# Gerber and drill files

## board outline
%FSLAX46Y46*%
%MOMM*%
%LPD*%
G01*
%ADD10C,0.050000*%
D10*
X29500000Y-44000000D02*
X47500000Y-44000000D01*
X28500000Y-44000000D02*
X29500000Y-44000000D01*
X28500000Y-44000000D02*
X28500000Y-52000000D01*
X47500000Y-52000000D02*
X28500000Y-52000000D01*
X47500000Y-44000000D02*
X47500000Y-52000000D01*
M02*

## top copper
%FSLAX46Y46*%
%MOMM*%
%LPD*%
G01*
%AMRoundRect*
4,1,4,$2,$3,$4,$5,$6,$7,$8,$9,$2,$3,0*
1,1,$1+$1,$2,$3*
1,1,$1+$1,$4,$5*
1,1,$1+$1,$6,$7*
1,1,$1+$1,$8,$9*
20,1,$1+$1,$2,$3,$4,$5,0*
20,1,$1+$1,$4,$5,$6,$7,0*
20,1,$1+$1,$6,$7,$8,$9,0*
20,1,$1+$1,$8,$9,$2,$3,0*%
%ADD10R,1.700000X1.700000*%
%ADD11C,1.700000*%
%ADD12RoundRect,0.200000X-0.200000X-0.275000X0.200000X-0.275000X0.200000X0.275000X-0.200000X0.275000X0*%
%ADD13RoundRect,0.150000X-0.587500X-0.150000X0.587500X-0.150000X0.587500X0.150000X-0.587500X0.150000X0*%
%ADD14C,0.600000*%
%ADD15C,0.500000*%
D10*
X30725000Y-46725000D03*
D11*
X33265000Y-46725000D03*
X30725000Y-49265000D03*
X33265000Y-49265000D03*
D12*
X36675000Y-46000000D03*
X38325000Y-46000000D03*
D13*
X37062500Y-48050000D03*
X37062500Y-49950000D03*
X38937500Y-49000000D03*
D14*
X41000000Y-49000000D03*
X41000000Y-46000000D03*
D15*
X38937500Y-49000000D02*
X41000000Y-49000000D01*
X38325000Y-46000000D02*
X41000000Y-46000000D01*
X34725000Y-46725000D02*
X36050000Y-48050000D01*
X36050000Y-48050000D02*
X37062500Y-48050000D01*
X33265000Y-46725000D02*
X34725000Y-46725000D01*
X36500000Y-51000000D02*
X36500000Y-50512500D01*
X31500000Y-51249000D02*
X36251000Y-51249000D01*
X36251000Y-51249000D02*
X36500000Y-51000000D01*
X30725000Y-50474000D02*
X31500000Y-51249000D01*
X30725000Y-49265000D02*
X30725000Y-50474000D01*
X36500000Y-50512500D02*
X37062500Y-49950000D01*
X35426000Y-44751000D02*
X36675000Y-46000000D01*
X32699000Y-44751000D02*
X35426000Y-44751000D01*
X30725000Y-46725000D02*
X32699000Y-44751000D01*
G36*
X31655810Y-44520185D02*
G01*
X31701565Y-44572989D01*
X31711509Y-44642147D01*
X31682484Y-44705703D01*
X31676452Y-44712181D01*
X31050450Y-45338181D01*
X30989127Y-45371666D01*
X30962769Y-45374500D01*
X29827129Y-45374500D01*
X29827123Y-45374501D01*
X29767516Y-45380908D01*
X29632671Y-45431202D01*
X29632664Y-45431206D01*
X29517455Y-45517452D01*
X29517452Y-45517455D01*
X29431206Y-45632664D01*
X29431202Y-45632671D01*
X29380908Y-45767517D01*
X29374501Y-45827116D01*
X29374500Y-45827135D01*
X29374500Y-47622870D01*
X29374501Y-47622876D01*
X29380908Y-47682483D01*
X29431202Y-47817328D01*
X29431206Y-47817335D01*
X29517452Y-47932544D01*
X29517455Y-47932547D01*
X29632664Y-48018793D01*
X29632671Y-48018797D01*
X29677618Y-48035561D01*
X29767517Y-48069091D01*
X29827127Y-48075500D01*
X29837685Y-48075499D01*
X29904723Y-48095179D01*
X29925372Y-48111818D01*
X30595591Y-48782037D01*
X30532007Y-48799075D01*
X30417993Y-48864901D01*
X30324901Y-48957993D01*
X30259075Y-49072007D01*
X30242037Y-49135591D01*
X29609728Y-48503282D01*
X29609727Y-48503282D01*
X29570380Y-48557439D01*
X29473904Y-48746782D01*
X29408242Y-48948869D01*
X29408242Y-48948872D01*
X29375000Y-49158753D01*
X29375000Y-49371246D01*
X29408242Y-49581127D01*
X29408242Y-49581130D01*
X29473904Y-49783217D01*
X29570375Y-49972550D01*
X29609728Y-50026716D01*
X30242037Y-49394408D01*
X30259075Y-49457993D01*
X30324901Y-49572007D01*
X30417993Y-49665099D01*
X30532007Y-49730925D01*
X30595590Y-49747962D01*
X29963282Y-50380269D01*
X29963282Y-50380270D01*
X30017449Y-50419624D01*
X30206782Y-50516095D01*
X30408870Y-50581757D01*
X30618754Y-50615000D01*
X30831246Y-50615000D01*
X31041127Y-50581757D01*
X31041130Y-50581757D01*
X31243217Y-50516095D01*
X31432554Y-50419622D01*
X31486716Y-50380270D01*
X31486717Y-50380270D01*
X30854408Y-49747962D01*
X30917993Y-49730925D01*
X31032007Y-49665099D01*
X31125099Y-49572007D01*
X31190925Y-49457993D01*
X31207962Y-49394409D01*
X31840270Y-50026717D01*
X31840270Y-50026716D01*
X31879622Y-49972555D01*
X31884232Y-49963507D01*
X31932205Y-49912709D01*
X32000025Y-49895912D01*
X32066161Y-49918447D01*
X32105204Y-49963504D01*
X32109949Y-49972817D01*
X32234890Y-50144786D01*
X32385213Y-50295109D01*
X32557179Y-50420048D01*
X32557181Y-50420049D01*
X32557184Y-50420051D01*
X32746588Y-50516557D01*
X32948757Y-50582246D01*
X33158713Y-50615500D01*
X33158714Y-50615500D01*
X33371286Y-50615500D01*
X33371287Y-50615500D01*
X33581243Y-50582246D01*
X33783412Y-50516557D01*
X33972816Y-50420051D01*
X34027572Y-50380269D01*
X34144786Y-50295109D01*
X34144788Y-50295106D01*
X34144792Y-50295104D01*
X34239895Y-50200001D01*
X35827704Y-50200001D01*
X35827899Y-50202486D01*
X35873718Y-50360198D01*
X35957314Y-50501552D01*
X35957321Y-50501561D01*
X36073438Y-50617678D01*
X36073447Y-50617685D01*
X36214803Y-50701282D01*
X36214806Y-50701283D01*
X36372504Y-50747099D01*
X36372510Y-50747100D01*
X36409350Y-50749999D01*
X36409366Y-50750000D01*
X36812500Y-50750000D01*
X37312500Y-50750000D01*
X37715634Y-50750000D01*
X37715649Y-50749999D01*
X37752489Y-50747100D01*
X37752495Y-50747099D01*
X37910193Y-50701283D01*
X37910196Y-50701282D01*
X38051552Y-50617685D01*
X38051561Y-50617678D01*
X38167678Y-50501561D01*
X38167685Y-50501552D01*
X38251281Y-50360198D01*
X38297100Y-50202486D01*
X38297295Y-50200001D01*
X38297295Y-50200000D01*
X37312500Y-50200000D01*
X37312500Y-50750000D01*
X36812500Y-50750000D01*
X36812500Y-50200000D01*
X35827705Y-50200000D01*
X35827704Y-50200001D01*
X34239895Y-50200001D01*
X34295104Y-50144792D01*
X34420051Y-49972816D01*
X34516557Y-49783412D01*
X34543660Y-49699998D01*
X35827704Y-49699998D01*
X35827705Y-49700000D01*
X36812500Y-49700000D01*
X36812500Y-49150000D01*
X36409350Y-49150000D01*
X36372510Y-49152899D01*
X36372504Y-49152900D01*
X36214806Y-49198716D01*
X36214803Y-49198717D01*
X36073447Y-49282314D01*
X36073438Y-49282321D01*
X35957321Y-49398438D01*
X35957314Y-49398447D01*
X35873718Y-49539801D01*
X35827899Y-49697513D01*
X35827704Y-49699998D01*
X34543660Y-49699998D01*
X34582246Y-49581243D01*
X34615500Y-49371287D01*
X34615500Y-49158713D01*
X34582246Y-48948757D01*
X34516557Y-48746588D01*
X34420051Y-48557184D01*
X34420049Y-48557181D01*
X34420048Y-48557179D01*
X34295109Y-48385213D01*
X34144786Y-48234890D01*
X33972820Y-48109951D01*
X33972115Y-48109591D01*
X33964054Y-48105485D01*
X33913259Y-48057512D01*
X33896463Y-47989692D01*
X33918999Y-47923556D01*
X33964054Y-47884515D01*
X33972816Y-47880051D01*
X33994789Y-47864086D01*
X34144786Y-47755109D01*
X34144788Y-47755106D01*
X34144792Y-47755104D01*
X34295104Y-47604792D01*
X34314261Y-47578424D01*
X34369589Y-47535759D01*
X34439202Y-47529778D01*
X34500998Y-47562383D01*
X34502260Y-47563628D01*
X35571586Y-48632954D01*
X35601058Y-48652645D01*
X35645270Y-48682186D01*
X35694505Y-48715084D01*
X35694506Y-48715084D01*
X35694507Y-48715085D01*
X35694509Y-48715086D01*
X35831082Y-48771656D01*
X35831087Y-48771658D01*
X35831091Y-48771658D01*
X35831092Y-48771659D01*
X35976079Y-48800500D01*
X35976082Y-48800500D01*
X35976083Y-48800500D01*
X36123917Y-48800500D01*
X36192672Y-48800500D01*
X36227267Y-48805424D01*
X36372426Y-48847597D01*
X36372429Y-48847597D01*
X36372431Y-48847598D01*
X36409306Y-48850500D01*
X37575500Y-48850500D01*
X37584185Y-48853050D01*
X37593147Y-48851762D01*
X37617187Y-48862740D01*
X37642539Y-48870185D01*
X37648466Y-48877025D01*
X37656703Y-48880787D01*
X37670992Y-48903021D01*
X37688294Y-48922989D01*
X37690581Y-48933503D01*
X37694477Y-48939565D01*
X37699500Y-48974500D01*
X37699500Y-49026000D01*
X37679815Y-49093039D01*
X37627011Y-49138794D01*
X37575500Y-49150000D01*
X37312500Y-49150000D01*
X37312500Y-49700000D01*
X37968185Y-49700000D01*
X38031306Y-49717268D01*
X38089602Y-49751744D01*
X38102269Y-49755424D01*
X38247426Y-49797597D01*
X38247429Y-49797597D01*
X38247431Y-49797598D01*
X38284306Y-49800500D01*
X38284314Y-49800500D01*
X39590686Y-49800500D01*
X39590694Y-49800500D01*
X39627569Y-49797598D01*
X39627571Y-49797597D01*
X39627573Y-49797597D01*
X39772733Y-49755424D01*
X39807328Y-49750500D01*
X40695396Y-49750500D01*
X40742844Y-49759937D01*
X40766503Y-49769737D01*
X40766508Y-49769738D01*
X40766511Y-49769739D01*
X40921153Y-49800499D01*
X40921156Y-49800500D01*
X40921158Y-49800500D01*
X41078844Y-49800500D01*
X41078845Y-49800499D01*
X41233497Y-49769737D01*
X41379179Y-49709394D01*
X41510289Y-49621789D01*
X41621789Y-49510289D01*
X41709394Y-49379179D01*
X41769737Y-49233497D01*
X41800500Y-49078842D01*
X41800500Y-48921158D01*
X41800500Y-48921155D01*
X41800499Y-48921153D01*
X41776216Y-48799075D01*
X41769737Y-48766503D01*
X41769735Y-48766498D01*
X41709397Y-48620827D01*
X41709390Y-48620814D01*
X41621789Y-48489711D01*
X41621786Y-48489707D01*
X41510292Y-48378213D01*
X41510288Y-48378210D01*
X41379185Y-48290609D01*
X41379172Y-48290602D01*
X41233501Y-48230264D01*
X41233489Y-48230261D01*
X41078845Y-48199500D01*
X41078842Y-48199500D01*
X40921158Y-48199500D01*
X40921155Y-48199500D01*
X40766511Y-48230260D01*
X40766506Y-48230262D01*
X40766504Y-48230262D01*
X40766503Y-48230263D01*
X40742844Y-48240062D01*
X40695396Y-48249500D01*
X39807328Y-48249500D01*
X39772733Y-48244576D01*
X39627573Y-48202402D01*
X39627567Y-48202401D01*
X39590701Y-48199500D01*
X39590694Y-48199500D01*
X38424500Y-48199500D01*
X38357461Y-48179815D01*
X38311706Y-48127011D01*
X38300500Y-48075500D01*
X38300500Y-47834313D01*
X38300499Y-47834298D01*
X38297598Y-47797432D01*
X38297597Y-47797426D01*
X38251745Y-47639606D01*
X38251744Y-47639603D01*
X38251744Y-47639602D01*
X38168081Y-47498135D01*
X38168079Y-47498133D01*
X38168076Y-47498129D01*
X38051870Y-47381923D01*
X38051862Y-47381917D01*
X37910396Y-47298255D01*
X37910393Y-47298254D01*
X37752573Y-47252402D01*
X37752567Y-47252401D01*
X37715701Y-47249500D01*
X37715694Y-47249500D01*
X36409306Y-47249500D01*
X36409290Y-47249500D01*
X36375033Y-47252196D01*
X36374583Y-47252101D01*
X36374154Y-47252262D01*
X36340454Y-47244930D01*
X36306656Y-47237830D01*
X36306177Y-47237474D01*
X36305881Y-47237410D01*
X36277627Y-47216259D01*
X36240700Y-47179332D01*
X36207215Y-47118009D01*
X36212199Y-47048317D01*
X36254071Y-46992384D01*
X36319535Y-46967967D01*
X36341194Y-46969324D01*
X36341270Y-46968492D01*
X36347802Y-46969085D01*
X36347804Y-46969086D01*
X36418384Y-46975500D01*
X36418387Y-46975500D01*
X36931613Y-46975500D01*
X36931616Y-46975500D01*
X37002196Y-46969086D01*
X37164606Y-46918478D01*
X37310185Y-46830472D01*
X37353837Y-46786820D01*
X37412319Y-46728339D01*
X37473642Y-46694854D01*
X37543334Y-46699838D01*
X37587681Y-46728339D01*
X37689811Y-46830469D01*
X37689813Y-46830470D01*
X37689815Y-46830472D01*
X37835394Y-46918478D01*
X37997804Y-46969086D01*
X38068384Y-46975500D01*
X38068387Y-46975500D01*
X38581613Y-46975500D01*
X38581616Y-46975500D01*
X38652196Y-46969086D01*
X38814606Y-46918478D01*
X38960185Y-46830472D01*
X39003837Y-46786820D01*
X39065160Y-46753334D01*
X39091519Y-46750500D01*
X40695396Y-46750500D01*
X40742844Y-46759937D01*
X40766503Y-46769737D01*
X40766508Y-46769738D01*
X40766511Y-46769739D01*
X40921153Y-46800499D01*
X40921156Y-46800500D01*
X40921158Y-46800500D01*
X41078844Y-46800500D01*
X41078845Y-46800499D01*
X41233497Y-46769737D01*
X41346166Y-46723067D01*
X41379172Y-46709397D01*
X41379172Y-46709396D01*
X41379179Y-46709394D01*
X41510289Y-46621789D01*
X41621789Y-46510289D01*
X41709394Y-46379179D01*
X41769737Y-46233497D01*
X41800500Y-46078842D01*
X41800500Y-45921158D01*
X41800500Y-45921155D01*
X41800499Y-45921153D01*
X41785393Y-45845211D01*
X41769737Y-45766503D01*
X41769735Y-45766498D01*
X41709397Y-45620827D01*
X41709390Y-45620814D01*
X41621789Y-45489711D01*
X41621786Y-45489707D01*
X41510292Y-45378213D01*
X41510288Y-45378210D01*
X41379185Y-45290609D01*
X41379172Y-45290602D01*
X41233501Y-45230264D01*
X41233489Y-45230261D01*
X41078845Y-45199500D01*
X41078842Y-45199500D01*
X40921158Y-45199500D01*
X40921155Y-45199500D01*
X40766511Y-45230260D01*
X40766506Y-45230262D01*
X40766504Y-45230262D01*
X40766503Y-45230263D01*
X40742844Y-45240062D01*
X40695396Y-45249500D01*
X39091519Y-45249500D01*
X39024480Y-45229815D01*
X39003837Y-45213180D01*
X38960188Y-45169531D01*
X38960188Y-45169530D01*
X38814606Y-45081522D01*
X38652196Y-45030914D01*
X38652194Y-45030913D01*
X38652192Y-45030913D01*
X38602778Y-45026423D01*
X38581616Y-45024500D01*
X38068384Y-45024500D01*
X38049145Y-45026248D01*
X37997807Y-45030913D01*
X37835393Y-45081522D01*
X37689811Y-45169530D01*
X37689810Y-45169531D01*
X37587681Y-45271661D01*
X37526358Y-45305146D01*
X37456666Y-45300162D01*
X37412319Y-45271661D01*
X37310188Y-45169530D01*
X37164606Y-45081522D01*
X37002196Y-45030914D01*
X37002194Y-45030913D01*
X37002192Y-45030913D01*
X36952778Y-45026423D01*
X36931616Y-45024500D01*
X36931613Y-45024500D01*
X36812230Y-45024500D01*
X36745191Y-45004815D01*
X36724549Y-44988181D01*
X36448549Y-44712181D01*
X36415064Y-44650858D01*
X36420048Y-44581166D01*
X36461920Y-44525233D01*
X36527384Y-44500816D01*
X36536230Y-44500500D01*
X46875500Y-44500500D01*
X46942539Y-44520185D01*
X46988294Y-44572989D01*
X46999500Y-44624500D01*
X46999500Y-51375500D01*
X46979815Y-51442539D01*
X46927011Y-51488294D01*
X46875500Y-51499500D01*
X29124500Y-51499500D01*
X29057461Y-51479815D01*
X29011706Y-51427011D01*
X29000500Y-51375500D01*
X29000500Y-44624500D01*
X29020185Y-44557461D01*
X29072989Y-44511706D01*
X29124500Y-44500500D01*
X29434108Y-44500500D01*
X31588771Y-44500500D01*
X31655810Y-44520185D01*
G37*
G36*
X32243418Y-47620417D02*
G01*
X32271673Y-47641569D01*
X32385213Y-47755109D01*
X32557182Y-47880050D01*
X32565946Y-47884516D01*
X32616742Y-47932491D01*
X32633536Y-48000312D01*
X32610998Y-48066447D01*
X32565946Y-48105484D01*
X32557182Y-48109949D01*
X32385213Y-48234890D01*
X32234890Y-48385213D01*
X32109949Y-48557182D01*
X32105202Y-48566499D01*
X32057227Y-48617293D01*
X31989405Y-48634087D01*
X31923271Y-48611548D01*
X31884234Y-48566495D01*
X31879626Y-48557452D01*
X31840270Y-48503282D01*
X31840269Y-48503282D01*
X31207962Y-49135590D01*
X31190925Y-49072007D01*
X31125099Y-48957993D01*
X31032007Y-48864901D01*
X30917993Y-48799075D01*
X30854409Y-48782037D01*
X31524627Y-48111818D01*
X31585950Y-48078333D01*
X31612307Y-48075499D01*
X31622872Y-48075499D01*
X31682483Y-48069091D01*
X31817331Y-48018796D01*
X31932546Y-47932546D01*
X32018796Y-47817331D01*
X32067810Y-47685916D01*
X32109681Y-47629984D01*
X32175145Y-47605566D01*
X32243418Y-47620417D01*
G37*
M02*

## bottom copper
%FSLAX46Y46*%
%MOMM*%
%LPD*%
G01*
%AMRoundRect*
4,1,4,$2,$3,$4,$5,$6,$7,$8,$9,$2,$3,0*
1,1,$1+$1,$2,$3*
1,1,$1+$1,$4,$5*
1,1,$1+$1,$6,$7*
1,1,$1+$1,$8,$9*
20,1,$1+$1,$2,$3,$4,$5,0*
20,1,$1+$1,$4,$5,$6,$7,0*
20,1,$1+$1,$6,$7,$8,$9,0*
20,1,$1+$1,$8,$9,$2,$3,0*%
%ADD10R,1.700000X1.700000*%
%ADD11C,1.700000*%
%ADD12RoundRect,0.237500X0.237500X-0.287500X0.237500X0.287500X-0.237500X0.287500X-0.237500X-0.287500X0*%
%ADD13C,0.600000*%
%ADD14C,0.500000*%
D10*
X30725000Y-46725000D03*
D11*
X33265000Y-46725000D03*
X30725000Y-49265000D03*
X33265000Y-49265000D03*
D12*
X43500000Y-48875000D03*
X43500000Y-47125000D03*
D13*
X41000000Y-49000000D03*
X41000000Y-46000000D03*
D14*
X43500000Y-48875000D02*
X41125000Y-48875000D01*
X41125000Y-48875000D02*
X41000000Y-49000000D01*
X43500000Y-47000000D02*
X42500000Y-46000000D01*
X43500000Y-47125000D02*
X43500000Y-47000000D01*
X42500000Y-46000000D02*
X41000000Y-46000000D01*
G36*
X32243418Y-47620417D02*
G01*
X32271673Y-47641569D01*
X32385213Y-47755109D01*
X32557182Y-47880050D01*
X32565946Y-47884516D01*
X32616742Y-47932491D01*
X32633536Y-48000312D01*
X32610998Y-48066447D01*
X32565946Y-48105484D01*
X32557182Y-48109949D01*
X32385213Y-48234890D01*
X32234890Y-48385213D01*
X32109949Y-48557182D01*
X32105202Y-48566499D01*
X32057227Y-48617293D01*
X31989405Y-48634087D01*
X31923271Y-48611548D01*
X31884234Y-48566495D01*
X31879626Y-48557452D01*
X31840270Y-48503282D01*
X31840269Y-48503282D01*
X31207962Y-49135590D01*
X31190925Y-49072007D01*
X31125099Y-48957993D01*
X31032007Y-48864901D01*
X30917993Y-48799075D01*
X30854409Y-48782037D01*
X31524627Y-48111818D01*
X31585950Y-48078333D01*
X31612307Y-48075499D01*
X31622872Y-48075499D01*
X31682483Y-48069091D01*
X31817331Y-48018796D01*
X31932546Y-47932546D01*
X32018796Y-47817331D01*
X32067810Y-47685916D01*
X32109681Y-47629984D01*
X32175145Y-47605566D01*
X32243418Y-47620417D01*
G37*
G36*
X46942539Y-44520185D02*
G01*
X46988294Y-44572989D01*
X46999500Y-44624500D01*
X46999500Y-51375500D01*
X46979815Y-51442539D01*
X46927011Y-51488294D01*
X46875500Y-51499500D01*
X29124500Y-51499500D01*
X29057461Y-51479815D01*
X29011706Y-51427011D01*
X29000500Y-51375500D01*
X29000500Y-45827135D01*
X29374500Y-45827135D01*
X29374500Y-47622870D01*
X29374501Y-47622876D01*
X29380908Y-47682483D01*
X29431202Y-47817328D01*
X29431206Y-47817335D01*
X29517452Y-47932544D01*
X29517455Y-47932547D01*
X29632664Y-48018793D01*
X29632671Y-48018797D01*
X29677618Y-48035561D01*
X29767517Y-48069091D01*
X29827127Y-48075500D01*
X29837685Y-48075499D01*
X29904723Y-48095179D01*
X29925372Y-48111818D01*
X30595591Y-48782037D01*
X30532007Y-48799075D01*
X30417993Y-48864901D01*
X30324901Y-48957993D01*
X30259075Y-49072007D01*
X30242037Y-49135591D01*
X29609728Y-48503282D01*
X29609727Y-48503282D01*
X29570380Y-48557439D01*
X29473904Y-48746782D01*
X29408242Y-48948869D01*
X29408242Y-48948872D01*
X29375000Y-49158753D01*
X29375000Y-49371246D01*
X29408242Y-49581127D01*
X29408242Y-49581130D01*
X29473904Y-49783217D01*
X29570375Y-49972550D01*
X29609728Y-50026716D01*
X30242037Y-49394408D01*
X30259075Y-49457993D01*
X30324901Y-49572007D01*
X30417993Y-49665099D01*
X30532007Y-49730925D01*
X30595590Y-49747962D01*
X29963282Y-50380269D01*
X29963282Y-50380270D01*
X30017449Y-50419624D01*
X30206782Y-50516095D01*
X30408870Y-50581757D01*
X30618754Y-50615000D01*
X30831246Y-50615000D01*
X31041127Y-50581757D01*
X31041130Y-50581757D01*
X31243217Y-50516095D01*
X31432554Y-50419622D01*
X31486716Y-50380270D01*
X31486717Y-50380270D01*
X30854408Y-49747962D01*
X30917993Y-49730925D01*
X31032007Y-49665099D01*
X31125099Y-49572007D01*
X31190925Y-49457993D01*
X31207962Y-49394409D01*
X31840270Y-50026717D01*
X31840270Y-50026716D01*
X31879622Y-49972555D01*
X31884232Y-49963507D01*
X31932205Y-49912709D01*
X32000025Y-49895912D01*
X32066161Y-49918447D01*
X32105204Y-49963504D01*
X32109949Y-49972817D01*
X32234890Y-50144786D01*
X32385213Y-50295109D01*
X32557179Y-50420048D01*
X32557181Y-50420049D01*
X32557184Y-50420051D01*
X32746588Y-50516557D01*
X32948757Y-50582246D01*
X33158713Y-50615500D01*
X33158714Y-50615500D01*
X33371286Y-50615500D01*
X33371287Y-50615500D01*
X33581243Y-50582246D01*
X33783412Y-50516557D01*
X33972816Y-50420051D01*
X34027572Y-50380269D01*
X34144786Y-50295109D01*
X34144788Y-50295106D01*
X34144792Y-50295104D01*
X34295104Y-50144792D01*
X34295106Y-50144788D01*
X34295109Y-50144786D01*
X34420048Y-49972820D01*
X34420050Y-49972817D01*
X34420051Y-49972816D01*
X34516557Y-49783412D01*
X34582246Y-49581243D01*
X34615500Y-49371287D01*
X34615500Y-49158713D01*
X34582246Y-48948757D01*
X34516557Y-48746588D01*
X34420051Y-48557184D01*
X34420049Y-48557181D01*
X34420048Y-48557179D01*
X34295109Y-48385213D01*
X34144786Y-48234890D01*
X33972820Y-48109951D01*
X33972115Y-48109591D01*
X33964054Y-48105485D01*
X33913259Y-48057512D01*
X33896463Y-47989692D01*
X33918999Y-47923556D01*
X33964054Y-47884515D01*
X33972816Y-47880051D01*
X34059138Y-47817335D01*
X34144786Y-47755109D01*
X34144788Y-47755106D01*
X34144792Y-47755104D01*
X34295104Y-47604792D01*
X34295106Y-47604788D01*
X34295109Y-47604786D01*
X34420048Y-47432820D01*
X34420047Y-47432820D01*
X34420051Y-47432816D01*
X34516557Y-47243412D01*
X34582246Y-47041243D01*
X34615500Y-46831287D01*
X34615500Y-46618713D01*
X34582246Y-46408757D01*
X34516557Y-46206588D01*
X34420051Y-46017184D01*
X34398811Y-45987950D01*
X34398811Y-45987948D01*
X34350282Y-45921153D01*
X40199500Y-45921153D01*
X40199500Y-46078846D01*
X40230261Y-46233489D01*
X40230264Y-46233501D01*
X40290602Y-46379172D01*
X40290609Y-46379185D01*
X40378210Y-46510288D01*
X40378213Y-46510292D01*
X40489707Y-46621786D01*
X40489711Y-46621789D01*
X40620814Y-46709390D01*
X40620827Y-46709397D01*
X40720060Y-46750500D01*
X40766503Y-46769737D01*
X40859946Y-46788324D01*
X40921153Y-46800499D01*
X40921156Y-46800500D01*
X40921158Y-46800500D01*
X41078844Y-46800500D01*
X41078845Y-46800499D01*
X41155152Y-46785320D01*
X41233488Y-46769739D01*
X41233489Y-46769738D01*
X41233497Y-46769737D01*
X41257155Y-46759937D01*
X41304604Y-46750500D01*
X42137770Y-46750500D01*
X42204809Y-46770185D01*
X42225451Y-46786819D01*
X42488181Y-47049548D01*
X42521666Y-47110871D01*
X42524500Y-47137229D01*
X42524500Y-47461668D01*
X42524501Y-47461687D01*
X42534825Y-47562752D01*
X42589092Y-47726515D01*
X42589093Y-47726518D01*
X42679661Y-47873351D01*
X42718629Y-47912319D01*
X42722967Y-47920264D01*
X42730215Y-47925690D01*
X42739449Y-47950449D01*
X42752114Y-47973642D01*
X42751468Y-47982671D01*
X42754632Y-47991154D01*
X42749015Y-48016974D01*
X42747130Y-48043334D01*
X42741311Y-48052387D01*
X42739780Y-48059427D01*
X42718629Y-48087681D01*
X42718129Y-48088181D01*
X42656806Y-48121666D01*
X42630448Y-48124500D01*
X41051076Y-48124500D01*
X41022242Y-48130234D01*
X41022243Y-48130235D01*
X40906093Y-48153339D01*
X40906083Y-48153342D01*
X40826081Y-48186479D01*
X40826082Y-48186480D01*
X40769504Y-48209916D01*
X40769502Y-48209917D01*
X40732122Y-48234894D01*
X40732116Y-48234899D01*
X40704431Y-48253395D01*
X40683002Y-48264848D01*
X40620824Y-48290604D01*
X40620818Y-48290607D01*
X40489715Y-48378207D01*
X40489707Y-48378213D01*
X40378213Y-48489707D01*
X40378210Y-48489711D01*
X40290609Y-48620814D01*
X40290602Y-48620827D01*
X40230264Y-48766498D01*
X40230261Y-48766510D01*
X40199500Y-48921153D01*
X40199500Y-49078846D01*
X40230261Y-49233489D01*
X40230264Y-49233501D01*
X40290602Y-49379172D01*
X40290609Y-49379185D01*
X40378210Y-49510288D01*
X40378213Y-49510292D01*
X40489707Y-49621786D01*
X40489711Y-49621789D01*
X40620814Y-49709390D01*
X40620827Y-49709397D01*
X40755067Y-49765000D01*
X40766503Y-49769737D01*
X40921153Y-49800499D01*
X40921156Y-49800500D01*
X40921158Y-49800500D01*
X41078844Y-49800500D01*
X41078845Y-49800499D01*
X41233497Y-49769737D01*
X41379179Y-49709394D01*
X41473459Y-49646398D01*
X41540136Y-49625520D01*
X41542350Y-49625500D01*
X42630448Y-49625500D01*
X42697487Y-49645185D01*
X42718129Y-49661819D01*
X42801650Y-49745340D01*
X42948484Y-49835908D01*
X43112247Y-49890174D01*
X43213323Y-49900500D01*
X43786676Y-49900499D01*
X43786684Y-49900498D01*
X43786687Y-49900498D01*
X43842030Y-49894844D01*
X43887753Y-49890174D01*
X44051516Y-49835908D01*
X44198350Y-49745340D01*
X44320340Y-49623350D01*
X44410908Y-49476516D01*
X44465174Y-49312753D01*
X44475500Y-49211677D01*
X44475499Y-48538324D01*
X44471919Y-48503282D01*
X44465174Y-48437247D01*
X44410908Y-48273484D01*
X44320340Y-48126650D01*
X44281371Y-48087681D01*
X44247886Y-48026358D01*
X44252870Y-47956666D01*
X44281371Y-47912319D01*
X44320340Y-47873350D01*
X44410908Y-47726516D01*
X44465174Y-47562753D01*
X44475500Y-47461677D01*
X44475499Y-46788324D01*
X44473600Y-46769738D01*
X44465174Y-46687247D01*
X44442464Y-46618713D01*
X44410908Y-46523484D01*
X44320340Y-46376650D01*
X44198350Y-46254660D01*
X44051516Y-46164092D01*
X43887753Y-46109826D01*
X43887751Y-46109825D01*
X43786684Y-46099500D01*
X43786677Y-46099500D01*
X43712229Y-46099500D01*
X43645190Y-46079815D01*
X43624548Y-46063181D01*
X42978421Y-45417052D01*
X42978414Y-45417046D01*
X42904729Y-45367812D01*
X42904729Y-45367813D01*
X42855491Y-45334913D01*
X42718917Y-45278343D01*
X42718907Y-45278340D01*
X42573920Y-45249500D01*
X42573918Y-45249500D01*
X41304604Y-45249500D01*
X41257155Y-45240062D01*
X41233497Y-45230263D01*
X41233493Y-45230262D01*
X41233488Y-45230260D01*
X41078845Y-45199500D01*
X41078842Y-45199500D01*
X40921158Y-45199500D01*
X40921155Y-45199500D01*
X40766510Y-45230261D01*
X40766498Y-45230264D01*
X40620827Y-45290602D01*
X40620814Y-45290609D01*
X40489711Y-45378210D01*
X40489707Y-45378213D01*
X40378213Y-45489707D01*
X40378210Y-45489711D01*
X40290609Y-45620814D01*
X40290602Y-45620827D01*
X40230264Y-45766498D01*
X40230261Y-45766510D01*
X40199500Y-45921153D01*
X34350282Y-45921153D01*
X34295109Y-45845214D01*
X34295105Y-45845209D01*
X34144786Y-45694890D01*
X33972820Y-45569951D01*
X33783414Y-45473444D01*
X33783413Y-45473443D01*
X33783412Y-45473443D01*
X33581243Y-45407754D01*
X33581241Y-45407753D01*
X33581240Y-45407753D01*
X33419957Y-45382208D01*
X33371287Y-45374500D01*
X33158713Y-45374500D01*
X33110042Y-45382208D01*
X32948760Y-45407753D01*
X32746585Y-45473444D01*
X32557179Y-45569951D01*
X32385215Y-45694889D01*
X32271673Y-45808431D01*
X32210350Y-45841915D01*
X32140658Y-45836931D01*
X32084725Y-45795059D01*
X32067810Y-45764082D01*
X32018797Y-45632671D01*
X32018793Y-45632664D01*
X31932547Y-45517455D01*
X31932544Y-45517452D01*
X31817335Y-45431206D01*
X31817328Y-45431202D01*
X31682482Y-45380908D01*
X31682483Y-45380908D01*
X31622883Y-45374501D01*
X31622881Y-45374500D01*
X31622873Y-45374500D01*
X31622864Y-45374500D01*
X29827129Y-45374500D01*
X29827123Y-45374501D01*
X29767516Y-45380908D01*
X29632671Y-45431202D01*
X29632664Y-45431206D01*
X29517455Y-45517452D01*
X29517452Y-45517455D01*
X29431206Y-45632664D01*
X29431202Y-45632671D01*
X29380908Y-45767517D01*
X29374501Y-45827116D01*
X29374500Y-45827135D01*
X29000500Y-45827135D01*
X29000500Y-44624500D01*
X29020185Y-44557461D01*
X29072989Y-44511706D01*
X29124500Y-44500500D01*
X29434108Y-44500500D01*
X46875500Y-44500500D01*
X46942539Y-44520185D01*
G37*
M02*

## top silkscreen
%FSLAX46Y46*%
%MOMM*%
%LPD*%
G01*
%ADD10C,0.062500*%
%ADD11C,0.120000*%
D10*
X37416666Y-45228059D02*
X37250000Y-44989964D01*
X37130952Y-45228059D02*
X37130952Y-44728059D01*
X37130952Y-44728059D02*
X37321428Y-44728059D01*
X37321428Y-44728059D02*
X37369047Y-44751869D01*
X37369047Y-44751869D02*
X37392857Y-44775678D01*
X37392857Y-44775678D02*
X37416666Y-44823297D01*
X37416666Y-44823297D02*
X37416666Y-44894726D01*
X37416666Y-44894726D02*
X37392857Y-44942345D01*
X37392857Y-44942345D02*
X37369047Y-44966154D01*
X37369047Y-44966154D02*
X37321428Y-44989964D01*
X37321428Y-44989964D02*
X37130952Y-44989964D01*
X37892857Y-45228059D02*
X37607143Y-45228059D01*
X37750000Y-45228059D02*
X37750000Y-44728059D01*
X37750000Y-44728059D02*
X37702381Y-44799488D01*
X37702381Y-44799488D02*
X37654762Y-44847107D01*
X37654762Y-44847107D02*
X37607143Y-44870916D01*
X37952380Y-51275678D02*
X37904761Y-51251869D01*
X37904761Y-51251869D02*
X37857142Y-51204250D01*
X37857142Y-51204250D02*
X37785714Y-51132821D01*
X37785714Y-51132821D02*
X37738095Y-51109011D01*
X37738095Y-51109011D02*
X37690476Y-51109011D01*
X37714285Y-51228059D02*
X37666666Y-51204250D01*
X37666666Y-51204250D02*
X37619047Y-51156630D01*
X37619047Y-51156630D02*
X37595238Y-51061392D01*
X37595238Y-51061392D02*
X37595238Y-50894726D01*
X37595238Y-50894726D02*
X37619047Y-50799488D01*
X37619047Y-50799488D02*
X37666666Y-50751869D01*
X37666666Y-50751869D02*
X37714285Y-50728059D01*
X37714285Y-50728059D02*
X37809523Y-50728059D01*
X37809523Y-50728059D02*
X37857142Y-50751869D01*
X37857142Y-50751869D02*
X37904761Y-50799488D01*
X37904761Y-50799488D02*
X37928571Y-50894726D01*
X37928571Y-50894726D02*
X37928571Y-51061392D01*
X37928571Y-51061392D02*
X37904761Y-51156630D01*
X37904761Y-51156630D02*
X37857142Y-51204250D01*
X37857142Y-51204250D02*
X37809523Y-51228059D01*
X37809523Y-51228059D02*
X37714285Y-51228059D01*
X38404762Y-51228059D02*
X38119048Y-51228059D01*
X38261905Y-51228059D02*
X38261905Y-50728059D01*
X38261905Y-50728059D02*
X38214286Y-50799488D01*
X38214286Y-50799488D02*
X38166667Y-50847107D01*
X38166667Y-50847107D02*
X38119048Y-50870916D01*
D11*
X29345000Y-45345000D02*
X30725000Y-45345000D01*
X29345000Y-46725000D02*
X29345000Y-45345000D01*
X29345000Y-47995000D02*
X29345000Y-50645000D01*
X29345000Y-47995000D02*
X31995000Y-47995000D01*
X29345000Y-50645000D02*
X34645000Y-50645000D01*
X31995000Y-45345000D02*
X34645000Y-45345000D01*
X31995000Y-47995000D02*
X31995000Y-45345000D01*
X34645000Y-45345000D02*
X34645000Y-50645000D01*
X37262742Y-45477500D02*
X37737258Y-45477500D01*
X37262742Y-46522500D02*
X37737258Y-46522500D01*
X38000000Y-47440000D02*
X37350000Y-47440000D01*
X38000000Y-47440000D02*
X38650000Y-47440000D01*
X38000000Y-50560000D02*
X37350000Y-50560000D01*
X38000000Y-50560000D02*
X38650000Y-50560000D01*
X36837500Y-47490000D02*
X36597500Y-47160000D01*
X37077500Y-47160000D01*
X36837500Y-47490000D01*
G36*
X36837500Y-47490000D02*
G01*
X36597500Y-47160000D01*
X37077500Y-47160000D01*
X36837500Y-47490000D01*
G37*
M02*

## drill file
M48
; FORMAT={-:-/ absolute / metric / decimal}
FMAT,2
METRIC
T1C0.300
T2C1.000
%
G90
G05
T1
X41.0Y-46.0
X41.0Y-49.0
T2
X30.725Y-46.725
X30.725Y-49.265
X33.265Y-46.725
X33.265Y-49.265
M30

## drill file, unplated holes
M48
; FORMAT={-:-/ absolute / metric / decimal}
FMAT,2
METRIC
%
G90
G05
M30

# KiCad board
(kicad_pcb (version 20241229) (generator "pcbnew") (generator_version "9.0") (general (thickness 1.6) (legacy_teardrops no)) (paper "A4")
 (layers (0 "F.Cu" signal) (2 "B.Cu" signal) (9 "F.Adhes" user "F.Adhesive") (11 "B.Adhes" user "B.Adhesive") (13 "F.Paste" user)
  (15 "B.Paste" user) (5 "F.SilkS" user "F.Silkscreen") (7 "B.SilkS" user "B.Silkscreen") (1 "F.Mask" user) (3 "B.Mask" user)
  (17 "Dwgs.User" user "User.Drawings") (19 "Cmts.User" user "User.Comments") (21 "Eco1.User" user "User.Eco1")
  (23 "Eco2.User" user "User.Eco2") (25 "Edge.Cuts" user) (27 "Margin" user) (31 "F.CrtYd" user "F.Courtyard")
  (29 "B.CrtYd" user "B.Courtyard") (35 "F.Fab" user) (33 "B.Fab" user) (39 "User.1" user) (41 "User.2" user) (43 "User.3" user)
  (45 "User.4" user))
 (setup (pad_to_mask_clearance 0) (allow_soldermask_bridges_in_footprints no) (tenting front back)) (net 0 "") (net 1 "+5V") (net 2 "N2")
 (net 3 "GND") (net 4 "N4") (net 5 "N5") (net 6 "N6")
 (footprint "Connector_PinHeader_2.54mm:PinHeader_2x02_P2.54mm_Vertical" (layer "F.Cu") (at 30.725 46.725)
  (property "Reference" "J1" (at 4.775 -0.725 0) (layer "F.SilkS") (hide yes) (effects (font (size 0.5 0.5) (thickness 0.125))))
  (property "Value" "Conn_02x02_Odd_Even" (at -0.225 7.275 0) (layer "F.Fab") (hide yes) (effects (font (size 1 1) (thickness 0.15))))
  (fp_line (start -1.38 -1.38) (end 0 -1.38) (stroke (width 0.12) (type solid)) (layer "F.SilkS"))
  (fp_line (start -1.38 0) (end -1.38 -1.38) (stroke (width 0.12) (type solid)) (layer "F.SilkS"))
  (fp_line (start -1.38 1.27) (end -1.38 3.92) (stroke (width 0.12) (type solid)) (layer "F.SilkS"))
  (fp_line (start -1.38 1.27) (end 1.27 1.27) (stroke (width 0.12) (type solid)) (layer "F.SilkS"))
  (fp_line (start -1.38 3.92) (end 3.92 3.92) (stroke (width 0.12) (type solid)) (layer "F.SilkS"))
  (fp_line (start 1.27 -1.38) (end 3.92 -1.38) (stroke (width 0.12) (type solid)) (layer "F.SilkS"))
  (fp_line (start 1.27 1.27) (end 1.27 -1.38) (stroke (width 0.12) (type solid)) (layer "F.SilkS"))
  (fp_line (start 3.92 -1.38) (end 3.92 3.92) (stroke (width 0.12) (type solid)) (layer "F.SilkS"))
  (pad "1" thru_hole rect (at 0 0) (size 1.7 1.7) (drill 1) (layers "*.Cu" "*.Mask") (remove_unused_layers no) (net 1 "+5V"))
  (pad "2" thru_hole circle (at 2.54 0) (size 1.7 1.7) (drill 1) (layers "*.Cu" "*.Mask") (remove_unused_layers no) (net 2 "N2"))
  (pad "3" thru_hole circle (at 0 2.54) (size 1.7 1.7) (drill 1) (layers "*.Cu" "*.Mask") (remove_unused_layers no) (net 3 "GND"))
  (pad "4" thru_hole circle (at 2.54 2.54) (size 1.7 1.7) (drill 1) (layers "*.Cu" "*.Mask") (remove_unused_layers no) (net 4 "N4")))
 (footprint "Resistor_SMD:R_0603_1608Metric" (layer "F.Cu") (at 37.5 46)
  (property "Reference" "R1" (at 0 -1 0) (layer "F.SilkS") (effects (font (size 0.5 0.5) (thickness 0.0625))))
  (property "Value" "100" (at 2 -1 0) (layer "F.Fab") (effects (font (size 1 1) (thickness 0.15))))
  (fp_line (start -0.237258 -0.5225) (end 0.237258 -0.5225) (stroke (width 0.12) (type solid)) (layer "F.SilkS"))
  (fp_line (start -0.237258 0.5225) (end 0.237258 0.5225) (stroke (width 0.12) (type solid)) (layer "F.SilkS"))
  (pad "1" smd roundrect (at -0.825 0) (size 0.8 0.95) (layers "F.Cu" "F.Mask" "F.Paste") (roundrect_rratio 0.25) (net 1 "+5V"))
  (pad "2" smd roundrect (at 0.825 0) (size 0.8 0.95) (layers "F.Cu" "F.Mask" "F.Paste") (roundrect_rratio 0.25) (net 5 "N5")))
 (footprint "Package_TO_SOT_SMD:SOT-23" (layer "F.Cu") (at 38 49)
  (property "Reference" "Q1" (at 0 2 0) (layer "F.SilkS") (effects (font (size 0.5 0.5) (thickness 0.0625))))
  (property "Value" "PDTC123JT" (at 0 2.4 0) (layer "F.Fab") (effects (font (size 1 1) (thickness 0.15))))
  (fp_line (start 0 -1.56) (end -0.65 -1.56) (stroke (width 0.12) (type solid)) (layer "F.SilkS"))
  (fp_line (start 0 -1.56) (end 0.65 -1.56) (stroke (width 0.12) (type solid)) (layer "F.SilkS"))
  (fp_line (start 0 1.56) (end -0.65 1.56) (stroke (width 0.12) (type solid)) (layer "F.SilkS"))
  (fp_line (start 0 1.56) (end 0.65 1.56) (stroke (width 0.12) (type solid)) (layer "F.SilkS"))
  (fp_poly (pts (xy -1.1625 -1.51) (xy -1.4025 -1.84) (xy -0.9225 -1.84)) (stroke (width 0.12) (type solid)) (fill yes) (layer "F.SilkS"))
  (pad "1" smd roundrect (at -0.9375 -0.95) (size 1.475 0.6) (layers "F.Cu" "F.Mask" "F.Paste") (roundrect_rratio 0.25) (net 2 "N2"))
  (pad "2" smd roundrect (at -0.9375 0.95) (size 1.475 0.6) (layers "F.Cu" "F.Mask" "F.Paste") (roundrect_rratio 0.25) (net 3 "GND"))
  (pad "3" smd roundrect (at 0.9375 0) (size 1.475 0.6) (layers "F.Cu" "F.Mask" "F.Paste") (roundrect_rratio 0.25) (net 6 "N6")))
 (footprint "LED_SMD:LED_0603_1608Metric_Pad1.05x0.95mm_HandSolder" (layer "B.Cu") (at 43.5 48 90)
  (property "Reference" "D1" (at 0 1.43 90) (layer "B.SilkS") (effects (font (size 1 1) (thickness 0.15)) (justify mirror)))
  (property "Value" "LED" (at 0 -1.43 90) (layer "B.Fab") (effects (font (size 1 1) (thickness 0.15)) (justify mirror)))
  (pad "1" smd roundrect (at -0.875 0 90) (size 1.05 0.95) (layers "B.Cu" "B.Mask" "B.Paste") (roundrect_rratio 0.25) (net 6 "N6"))
  (pad "2" smd roundrect (at 0.875 0 90) (size 1.05 0.95) (layers "B.Cu" "B.Mask" "B.Paste") (roundrect_rratio 0.25) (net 5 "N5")))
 (gr_line (start 29.5 44) (end 47.5 44) (stroke (width 0.05) (type default)) (layer "Edge.Cuts"))
 (gr_line (start 28.5 44) (end 29.5 44) (stroke (width 0.05) (type default)) (layer "Edge.Cuts"))
 (gr_line (start 28.5 44) (end 28.5 52) (stroke (width 0.05) (type default)) (layer "Edge.Cuts"))
 (gr_line (start 47.5 52) (end 28.5 52) (stroke (width 0.05) (type default)) (layer "Edge.Cuts"))
 (gr_line (start 47.5 44) (end 47.5 52) (stroke (width 0.05) (type default)) (layer "Edge.Cuts"))
 (segment (start 38.325 46) (end 41 46) (width 0.5) (layer "F.Cu") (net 5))
 (via (at 41 46) (size 0.6) (drill 0.3) (layers "F.Cu" "B.Cu") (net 5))
 (segment (start 42.5 46) (end 41 46) (width 0.5) (layer "B.Cu") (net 5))
 (segment (start 43.5 47) (end 42.5 46) (width 0.5) (layer "B.Cu") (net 5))
 (segment (start 43.5 47.125) (end 43.5 47) (width 0.5) (layer "B.Cu") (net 5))
 (segment (start 38.9375 49) (end 41 49) (width 0.5) (layer "F.Cu") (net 6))
 (via (at 41 49) (size 0.6) (drill 0.3) (layers "F.Cu" "B.Cu") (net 6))
 (segment (start 43.5 48.875) (end 41.125 48.875) (width 0.5) (layer "B.Cu") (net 6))
 (segment (start 41.125 48.875) (end 41 49) (width 0.5) (layer "B.Cu") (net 6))
 (segment (start 34.725 46.725) (end 36.05 48.05) (width 0.5) (layer "F.Cu") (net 2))
 (segment (start 36.05 48.05) (end 37.0625 48.05) (width 0.5) (layer "F.Cu") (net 2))
 (segment (start 33.265 46.725) (end 34.725 46.725) (width 0.5) (layer "F.Cu") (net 2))
 (segment (start 36.5 51) (end 36.5 50.5125) (width 0.5) (layer "F.Cu") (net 3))
 (segment (start 31.5 51.249) (end 36.251 51.249) (width 0.5) (layer "F.Cu") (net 3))
 (segment (start 36.251 51.249) (end 36.5 51) (width 0.5) (layer "F.Cu") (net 3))
 (segment (start 30.725 50.474) (end 31.5 51.249) (width 0.5) (layer "F.Cu") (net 3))
 (segment (start 30.725 49.265) (end 30.725 50.474) (width 0.5) (layer "F.Cu") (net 3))
 (segment (start 36.5 50.5125) (end 37.0625 49.95) (width 0.5) (layer "F.Cu") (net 3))
 (segment (start 35.426 44.751) (end 36.675 46) (width 0.5) (layer "F.Cu") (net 1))
 (segment (start 32.699 44.751) (end 35.426 44.751) (width 0.5) (layer "F.Cu") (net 1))
 (segment (start 30.725 46.725) (end 32.699 44.751) (width 0.5) (layer "F.Cu") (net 1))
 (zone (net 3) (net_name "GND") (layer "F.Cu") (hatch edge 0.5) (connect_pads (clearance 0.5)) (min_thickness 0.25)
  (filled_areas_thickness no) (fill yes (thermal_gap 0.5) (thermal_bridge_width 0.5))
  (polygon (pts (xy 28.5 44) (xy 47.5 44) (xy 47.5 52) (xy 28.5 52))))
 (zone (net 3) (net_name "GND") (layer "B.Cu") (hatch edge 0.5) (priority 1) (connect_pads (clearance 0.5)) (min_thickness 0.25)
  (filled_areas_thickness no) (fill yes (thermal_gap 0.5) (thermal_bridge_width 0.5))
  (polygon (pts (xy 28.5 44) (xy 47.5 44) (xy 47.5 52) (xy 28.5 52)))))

